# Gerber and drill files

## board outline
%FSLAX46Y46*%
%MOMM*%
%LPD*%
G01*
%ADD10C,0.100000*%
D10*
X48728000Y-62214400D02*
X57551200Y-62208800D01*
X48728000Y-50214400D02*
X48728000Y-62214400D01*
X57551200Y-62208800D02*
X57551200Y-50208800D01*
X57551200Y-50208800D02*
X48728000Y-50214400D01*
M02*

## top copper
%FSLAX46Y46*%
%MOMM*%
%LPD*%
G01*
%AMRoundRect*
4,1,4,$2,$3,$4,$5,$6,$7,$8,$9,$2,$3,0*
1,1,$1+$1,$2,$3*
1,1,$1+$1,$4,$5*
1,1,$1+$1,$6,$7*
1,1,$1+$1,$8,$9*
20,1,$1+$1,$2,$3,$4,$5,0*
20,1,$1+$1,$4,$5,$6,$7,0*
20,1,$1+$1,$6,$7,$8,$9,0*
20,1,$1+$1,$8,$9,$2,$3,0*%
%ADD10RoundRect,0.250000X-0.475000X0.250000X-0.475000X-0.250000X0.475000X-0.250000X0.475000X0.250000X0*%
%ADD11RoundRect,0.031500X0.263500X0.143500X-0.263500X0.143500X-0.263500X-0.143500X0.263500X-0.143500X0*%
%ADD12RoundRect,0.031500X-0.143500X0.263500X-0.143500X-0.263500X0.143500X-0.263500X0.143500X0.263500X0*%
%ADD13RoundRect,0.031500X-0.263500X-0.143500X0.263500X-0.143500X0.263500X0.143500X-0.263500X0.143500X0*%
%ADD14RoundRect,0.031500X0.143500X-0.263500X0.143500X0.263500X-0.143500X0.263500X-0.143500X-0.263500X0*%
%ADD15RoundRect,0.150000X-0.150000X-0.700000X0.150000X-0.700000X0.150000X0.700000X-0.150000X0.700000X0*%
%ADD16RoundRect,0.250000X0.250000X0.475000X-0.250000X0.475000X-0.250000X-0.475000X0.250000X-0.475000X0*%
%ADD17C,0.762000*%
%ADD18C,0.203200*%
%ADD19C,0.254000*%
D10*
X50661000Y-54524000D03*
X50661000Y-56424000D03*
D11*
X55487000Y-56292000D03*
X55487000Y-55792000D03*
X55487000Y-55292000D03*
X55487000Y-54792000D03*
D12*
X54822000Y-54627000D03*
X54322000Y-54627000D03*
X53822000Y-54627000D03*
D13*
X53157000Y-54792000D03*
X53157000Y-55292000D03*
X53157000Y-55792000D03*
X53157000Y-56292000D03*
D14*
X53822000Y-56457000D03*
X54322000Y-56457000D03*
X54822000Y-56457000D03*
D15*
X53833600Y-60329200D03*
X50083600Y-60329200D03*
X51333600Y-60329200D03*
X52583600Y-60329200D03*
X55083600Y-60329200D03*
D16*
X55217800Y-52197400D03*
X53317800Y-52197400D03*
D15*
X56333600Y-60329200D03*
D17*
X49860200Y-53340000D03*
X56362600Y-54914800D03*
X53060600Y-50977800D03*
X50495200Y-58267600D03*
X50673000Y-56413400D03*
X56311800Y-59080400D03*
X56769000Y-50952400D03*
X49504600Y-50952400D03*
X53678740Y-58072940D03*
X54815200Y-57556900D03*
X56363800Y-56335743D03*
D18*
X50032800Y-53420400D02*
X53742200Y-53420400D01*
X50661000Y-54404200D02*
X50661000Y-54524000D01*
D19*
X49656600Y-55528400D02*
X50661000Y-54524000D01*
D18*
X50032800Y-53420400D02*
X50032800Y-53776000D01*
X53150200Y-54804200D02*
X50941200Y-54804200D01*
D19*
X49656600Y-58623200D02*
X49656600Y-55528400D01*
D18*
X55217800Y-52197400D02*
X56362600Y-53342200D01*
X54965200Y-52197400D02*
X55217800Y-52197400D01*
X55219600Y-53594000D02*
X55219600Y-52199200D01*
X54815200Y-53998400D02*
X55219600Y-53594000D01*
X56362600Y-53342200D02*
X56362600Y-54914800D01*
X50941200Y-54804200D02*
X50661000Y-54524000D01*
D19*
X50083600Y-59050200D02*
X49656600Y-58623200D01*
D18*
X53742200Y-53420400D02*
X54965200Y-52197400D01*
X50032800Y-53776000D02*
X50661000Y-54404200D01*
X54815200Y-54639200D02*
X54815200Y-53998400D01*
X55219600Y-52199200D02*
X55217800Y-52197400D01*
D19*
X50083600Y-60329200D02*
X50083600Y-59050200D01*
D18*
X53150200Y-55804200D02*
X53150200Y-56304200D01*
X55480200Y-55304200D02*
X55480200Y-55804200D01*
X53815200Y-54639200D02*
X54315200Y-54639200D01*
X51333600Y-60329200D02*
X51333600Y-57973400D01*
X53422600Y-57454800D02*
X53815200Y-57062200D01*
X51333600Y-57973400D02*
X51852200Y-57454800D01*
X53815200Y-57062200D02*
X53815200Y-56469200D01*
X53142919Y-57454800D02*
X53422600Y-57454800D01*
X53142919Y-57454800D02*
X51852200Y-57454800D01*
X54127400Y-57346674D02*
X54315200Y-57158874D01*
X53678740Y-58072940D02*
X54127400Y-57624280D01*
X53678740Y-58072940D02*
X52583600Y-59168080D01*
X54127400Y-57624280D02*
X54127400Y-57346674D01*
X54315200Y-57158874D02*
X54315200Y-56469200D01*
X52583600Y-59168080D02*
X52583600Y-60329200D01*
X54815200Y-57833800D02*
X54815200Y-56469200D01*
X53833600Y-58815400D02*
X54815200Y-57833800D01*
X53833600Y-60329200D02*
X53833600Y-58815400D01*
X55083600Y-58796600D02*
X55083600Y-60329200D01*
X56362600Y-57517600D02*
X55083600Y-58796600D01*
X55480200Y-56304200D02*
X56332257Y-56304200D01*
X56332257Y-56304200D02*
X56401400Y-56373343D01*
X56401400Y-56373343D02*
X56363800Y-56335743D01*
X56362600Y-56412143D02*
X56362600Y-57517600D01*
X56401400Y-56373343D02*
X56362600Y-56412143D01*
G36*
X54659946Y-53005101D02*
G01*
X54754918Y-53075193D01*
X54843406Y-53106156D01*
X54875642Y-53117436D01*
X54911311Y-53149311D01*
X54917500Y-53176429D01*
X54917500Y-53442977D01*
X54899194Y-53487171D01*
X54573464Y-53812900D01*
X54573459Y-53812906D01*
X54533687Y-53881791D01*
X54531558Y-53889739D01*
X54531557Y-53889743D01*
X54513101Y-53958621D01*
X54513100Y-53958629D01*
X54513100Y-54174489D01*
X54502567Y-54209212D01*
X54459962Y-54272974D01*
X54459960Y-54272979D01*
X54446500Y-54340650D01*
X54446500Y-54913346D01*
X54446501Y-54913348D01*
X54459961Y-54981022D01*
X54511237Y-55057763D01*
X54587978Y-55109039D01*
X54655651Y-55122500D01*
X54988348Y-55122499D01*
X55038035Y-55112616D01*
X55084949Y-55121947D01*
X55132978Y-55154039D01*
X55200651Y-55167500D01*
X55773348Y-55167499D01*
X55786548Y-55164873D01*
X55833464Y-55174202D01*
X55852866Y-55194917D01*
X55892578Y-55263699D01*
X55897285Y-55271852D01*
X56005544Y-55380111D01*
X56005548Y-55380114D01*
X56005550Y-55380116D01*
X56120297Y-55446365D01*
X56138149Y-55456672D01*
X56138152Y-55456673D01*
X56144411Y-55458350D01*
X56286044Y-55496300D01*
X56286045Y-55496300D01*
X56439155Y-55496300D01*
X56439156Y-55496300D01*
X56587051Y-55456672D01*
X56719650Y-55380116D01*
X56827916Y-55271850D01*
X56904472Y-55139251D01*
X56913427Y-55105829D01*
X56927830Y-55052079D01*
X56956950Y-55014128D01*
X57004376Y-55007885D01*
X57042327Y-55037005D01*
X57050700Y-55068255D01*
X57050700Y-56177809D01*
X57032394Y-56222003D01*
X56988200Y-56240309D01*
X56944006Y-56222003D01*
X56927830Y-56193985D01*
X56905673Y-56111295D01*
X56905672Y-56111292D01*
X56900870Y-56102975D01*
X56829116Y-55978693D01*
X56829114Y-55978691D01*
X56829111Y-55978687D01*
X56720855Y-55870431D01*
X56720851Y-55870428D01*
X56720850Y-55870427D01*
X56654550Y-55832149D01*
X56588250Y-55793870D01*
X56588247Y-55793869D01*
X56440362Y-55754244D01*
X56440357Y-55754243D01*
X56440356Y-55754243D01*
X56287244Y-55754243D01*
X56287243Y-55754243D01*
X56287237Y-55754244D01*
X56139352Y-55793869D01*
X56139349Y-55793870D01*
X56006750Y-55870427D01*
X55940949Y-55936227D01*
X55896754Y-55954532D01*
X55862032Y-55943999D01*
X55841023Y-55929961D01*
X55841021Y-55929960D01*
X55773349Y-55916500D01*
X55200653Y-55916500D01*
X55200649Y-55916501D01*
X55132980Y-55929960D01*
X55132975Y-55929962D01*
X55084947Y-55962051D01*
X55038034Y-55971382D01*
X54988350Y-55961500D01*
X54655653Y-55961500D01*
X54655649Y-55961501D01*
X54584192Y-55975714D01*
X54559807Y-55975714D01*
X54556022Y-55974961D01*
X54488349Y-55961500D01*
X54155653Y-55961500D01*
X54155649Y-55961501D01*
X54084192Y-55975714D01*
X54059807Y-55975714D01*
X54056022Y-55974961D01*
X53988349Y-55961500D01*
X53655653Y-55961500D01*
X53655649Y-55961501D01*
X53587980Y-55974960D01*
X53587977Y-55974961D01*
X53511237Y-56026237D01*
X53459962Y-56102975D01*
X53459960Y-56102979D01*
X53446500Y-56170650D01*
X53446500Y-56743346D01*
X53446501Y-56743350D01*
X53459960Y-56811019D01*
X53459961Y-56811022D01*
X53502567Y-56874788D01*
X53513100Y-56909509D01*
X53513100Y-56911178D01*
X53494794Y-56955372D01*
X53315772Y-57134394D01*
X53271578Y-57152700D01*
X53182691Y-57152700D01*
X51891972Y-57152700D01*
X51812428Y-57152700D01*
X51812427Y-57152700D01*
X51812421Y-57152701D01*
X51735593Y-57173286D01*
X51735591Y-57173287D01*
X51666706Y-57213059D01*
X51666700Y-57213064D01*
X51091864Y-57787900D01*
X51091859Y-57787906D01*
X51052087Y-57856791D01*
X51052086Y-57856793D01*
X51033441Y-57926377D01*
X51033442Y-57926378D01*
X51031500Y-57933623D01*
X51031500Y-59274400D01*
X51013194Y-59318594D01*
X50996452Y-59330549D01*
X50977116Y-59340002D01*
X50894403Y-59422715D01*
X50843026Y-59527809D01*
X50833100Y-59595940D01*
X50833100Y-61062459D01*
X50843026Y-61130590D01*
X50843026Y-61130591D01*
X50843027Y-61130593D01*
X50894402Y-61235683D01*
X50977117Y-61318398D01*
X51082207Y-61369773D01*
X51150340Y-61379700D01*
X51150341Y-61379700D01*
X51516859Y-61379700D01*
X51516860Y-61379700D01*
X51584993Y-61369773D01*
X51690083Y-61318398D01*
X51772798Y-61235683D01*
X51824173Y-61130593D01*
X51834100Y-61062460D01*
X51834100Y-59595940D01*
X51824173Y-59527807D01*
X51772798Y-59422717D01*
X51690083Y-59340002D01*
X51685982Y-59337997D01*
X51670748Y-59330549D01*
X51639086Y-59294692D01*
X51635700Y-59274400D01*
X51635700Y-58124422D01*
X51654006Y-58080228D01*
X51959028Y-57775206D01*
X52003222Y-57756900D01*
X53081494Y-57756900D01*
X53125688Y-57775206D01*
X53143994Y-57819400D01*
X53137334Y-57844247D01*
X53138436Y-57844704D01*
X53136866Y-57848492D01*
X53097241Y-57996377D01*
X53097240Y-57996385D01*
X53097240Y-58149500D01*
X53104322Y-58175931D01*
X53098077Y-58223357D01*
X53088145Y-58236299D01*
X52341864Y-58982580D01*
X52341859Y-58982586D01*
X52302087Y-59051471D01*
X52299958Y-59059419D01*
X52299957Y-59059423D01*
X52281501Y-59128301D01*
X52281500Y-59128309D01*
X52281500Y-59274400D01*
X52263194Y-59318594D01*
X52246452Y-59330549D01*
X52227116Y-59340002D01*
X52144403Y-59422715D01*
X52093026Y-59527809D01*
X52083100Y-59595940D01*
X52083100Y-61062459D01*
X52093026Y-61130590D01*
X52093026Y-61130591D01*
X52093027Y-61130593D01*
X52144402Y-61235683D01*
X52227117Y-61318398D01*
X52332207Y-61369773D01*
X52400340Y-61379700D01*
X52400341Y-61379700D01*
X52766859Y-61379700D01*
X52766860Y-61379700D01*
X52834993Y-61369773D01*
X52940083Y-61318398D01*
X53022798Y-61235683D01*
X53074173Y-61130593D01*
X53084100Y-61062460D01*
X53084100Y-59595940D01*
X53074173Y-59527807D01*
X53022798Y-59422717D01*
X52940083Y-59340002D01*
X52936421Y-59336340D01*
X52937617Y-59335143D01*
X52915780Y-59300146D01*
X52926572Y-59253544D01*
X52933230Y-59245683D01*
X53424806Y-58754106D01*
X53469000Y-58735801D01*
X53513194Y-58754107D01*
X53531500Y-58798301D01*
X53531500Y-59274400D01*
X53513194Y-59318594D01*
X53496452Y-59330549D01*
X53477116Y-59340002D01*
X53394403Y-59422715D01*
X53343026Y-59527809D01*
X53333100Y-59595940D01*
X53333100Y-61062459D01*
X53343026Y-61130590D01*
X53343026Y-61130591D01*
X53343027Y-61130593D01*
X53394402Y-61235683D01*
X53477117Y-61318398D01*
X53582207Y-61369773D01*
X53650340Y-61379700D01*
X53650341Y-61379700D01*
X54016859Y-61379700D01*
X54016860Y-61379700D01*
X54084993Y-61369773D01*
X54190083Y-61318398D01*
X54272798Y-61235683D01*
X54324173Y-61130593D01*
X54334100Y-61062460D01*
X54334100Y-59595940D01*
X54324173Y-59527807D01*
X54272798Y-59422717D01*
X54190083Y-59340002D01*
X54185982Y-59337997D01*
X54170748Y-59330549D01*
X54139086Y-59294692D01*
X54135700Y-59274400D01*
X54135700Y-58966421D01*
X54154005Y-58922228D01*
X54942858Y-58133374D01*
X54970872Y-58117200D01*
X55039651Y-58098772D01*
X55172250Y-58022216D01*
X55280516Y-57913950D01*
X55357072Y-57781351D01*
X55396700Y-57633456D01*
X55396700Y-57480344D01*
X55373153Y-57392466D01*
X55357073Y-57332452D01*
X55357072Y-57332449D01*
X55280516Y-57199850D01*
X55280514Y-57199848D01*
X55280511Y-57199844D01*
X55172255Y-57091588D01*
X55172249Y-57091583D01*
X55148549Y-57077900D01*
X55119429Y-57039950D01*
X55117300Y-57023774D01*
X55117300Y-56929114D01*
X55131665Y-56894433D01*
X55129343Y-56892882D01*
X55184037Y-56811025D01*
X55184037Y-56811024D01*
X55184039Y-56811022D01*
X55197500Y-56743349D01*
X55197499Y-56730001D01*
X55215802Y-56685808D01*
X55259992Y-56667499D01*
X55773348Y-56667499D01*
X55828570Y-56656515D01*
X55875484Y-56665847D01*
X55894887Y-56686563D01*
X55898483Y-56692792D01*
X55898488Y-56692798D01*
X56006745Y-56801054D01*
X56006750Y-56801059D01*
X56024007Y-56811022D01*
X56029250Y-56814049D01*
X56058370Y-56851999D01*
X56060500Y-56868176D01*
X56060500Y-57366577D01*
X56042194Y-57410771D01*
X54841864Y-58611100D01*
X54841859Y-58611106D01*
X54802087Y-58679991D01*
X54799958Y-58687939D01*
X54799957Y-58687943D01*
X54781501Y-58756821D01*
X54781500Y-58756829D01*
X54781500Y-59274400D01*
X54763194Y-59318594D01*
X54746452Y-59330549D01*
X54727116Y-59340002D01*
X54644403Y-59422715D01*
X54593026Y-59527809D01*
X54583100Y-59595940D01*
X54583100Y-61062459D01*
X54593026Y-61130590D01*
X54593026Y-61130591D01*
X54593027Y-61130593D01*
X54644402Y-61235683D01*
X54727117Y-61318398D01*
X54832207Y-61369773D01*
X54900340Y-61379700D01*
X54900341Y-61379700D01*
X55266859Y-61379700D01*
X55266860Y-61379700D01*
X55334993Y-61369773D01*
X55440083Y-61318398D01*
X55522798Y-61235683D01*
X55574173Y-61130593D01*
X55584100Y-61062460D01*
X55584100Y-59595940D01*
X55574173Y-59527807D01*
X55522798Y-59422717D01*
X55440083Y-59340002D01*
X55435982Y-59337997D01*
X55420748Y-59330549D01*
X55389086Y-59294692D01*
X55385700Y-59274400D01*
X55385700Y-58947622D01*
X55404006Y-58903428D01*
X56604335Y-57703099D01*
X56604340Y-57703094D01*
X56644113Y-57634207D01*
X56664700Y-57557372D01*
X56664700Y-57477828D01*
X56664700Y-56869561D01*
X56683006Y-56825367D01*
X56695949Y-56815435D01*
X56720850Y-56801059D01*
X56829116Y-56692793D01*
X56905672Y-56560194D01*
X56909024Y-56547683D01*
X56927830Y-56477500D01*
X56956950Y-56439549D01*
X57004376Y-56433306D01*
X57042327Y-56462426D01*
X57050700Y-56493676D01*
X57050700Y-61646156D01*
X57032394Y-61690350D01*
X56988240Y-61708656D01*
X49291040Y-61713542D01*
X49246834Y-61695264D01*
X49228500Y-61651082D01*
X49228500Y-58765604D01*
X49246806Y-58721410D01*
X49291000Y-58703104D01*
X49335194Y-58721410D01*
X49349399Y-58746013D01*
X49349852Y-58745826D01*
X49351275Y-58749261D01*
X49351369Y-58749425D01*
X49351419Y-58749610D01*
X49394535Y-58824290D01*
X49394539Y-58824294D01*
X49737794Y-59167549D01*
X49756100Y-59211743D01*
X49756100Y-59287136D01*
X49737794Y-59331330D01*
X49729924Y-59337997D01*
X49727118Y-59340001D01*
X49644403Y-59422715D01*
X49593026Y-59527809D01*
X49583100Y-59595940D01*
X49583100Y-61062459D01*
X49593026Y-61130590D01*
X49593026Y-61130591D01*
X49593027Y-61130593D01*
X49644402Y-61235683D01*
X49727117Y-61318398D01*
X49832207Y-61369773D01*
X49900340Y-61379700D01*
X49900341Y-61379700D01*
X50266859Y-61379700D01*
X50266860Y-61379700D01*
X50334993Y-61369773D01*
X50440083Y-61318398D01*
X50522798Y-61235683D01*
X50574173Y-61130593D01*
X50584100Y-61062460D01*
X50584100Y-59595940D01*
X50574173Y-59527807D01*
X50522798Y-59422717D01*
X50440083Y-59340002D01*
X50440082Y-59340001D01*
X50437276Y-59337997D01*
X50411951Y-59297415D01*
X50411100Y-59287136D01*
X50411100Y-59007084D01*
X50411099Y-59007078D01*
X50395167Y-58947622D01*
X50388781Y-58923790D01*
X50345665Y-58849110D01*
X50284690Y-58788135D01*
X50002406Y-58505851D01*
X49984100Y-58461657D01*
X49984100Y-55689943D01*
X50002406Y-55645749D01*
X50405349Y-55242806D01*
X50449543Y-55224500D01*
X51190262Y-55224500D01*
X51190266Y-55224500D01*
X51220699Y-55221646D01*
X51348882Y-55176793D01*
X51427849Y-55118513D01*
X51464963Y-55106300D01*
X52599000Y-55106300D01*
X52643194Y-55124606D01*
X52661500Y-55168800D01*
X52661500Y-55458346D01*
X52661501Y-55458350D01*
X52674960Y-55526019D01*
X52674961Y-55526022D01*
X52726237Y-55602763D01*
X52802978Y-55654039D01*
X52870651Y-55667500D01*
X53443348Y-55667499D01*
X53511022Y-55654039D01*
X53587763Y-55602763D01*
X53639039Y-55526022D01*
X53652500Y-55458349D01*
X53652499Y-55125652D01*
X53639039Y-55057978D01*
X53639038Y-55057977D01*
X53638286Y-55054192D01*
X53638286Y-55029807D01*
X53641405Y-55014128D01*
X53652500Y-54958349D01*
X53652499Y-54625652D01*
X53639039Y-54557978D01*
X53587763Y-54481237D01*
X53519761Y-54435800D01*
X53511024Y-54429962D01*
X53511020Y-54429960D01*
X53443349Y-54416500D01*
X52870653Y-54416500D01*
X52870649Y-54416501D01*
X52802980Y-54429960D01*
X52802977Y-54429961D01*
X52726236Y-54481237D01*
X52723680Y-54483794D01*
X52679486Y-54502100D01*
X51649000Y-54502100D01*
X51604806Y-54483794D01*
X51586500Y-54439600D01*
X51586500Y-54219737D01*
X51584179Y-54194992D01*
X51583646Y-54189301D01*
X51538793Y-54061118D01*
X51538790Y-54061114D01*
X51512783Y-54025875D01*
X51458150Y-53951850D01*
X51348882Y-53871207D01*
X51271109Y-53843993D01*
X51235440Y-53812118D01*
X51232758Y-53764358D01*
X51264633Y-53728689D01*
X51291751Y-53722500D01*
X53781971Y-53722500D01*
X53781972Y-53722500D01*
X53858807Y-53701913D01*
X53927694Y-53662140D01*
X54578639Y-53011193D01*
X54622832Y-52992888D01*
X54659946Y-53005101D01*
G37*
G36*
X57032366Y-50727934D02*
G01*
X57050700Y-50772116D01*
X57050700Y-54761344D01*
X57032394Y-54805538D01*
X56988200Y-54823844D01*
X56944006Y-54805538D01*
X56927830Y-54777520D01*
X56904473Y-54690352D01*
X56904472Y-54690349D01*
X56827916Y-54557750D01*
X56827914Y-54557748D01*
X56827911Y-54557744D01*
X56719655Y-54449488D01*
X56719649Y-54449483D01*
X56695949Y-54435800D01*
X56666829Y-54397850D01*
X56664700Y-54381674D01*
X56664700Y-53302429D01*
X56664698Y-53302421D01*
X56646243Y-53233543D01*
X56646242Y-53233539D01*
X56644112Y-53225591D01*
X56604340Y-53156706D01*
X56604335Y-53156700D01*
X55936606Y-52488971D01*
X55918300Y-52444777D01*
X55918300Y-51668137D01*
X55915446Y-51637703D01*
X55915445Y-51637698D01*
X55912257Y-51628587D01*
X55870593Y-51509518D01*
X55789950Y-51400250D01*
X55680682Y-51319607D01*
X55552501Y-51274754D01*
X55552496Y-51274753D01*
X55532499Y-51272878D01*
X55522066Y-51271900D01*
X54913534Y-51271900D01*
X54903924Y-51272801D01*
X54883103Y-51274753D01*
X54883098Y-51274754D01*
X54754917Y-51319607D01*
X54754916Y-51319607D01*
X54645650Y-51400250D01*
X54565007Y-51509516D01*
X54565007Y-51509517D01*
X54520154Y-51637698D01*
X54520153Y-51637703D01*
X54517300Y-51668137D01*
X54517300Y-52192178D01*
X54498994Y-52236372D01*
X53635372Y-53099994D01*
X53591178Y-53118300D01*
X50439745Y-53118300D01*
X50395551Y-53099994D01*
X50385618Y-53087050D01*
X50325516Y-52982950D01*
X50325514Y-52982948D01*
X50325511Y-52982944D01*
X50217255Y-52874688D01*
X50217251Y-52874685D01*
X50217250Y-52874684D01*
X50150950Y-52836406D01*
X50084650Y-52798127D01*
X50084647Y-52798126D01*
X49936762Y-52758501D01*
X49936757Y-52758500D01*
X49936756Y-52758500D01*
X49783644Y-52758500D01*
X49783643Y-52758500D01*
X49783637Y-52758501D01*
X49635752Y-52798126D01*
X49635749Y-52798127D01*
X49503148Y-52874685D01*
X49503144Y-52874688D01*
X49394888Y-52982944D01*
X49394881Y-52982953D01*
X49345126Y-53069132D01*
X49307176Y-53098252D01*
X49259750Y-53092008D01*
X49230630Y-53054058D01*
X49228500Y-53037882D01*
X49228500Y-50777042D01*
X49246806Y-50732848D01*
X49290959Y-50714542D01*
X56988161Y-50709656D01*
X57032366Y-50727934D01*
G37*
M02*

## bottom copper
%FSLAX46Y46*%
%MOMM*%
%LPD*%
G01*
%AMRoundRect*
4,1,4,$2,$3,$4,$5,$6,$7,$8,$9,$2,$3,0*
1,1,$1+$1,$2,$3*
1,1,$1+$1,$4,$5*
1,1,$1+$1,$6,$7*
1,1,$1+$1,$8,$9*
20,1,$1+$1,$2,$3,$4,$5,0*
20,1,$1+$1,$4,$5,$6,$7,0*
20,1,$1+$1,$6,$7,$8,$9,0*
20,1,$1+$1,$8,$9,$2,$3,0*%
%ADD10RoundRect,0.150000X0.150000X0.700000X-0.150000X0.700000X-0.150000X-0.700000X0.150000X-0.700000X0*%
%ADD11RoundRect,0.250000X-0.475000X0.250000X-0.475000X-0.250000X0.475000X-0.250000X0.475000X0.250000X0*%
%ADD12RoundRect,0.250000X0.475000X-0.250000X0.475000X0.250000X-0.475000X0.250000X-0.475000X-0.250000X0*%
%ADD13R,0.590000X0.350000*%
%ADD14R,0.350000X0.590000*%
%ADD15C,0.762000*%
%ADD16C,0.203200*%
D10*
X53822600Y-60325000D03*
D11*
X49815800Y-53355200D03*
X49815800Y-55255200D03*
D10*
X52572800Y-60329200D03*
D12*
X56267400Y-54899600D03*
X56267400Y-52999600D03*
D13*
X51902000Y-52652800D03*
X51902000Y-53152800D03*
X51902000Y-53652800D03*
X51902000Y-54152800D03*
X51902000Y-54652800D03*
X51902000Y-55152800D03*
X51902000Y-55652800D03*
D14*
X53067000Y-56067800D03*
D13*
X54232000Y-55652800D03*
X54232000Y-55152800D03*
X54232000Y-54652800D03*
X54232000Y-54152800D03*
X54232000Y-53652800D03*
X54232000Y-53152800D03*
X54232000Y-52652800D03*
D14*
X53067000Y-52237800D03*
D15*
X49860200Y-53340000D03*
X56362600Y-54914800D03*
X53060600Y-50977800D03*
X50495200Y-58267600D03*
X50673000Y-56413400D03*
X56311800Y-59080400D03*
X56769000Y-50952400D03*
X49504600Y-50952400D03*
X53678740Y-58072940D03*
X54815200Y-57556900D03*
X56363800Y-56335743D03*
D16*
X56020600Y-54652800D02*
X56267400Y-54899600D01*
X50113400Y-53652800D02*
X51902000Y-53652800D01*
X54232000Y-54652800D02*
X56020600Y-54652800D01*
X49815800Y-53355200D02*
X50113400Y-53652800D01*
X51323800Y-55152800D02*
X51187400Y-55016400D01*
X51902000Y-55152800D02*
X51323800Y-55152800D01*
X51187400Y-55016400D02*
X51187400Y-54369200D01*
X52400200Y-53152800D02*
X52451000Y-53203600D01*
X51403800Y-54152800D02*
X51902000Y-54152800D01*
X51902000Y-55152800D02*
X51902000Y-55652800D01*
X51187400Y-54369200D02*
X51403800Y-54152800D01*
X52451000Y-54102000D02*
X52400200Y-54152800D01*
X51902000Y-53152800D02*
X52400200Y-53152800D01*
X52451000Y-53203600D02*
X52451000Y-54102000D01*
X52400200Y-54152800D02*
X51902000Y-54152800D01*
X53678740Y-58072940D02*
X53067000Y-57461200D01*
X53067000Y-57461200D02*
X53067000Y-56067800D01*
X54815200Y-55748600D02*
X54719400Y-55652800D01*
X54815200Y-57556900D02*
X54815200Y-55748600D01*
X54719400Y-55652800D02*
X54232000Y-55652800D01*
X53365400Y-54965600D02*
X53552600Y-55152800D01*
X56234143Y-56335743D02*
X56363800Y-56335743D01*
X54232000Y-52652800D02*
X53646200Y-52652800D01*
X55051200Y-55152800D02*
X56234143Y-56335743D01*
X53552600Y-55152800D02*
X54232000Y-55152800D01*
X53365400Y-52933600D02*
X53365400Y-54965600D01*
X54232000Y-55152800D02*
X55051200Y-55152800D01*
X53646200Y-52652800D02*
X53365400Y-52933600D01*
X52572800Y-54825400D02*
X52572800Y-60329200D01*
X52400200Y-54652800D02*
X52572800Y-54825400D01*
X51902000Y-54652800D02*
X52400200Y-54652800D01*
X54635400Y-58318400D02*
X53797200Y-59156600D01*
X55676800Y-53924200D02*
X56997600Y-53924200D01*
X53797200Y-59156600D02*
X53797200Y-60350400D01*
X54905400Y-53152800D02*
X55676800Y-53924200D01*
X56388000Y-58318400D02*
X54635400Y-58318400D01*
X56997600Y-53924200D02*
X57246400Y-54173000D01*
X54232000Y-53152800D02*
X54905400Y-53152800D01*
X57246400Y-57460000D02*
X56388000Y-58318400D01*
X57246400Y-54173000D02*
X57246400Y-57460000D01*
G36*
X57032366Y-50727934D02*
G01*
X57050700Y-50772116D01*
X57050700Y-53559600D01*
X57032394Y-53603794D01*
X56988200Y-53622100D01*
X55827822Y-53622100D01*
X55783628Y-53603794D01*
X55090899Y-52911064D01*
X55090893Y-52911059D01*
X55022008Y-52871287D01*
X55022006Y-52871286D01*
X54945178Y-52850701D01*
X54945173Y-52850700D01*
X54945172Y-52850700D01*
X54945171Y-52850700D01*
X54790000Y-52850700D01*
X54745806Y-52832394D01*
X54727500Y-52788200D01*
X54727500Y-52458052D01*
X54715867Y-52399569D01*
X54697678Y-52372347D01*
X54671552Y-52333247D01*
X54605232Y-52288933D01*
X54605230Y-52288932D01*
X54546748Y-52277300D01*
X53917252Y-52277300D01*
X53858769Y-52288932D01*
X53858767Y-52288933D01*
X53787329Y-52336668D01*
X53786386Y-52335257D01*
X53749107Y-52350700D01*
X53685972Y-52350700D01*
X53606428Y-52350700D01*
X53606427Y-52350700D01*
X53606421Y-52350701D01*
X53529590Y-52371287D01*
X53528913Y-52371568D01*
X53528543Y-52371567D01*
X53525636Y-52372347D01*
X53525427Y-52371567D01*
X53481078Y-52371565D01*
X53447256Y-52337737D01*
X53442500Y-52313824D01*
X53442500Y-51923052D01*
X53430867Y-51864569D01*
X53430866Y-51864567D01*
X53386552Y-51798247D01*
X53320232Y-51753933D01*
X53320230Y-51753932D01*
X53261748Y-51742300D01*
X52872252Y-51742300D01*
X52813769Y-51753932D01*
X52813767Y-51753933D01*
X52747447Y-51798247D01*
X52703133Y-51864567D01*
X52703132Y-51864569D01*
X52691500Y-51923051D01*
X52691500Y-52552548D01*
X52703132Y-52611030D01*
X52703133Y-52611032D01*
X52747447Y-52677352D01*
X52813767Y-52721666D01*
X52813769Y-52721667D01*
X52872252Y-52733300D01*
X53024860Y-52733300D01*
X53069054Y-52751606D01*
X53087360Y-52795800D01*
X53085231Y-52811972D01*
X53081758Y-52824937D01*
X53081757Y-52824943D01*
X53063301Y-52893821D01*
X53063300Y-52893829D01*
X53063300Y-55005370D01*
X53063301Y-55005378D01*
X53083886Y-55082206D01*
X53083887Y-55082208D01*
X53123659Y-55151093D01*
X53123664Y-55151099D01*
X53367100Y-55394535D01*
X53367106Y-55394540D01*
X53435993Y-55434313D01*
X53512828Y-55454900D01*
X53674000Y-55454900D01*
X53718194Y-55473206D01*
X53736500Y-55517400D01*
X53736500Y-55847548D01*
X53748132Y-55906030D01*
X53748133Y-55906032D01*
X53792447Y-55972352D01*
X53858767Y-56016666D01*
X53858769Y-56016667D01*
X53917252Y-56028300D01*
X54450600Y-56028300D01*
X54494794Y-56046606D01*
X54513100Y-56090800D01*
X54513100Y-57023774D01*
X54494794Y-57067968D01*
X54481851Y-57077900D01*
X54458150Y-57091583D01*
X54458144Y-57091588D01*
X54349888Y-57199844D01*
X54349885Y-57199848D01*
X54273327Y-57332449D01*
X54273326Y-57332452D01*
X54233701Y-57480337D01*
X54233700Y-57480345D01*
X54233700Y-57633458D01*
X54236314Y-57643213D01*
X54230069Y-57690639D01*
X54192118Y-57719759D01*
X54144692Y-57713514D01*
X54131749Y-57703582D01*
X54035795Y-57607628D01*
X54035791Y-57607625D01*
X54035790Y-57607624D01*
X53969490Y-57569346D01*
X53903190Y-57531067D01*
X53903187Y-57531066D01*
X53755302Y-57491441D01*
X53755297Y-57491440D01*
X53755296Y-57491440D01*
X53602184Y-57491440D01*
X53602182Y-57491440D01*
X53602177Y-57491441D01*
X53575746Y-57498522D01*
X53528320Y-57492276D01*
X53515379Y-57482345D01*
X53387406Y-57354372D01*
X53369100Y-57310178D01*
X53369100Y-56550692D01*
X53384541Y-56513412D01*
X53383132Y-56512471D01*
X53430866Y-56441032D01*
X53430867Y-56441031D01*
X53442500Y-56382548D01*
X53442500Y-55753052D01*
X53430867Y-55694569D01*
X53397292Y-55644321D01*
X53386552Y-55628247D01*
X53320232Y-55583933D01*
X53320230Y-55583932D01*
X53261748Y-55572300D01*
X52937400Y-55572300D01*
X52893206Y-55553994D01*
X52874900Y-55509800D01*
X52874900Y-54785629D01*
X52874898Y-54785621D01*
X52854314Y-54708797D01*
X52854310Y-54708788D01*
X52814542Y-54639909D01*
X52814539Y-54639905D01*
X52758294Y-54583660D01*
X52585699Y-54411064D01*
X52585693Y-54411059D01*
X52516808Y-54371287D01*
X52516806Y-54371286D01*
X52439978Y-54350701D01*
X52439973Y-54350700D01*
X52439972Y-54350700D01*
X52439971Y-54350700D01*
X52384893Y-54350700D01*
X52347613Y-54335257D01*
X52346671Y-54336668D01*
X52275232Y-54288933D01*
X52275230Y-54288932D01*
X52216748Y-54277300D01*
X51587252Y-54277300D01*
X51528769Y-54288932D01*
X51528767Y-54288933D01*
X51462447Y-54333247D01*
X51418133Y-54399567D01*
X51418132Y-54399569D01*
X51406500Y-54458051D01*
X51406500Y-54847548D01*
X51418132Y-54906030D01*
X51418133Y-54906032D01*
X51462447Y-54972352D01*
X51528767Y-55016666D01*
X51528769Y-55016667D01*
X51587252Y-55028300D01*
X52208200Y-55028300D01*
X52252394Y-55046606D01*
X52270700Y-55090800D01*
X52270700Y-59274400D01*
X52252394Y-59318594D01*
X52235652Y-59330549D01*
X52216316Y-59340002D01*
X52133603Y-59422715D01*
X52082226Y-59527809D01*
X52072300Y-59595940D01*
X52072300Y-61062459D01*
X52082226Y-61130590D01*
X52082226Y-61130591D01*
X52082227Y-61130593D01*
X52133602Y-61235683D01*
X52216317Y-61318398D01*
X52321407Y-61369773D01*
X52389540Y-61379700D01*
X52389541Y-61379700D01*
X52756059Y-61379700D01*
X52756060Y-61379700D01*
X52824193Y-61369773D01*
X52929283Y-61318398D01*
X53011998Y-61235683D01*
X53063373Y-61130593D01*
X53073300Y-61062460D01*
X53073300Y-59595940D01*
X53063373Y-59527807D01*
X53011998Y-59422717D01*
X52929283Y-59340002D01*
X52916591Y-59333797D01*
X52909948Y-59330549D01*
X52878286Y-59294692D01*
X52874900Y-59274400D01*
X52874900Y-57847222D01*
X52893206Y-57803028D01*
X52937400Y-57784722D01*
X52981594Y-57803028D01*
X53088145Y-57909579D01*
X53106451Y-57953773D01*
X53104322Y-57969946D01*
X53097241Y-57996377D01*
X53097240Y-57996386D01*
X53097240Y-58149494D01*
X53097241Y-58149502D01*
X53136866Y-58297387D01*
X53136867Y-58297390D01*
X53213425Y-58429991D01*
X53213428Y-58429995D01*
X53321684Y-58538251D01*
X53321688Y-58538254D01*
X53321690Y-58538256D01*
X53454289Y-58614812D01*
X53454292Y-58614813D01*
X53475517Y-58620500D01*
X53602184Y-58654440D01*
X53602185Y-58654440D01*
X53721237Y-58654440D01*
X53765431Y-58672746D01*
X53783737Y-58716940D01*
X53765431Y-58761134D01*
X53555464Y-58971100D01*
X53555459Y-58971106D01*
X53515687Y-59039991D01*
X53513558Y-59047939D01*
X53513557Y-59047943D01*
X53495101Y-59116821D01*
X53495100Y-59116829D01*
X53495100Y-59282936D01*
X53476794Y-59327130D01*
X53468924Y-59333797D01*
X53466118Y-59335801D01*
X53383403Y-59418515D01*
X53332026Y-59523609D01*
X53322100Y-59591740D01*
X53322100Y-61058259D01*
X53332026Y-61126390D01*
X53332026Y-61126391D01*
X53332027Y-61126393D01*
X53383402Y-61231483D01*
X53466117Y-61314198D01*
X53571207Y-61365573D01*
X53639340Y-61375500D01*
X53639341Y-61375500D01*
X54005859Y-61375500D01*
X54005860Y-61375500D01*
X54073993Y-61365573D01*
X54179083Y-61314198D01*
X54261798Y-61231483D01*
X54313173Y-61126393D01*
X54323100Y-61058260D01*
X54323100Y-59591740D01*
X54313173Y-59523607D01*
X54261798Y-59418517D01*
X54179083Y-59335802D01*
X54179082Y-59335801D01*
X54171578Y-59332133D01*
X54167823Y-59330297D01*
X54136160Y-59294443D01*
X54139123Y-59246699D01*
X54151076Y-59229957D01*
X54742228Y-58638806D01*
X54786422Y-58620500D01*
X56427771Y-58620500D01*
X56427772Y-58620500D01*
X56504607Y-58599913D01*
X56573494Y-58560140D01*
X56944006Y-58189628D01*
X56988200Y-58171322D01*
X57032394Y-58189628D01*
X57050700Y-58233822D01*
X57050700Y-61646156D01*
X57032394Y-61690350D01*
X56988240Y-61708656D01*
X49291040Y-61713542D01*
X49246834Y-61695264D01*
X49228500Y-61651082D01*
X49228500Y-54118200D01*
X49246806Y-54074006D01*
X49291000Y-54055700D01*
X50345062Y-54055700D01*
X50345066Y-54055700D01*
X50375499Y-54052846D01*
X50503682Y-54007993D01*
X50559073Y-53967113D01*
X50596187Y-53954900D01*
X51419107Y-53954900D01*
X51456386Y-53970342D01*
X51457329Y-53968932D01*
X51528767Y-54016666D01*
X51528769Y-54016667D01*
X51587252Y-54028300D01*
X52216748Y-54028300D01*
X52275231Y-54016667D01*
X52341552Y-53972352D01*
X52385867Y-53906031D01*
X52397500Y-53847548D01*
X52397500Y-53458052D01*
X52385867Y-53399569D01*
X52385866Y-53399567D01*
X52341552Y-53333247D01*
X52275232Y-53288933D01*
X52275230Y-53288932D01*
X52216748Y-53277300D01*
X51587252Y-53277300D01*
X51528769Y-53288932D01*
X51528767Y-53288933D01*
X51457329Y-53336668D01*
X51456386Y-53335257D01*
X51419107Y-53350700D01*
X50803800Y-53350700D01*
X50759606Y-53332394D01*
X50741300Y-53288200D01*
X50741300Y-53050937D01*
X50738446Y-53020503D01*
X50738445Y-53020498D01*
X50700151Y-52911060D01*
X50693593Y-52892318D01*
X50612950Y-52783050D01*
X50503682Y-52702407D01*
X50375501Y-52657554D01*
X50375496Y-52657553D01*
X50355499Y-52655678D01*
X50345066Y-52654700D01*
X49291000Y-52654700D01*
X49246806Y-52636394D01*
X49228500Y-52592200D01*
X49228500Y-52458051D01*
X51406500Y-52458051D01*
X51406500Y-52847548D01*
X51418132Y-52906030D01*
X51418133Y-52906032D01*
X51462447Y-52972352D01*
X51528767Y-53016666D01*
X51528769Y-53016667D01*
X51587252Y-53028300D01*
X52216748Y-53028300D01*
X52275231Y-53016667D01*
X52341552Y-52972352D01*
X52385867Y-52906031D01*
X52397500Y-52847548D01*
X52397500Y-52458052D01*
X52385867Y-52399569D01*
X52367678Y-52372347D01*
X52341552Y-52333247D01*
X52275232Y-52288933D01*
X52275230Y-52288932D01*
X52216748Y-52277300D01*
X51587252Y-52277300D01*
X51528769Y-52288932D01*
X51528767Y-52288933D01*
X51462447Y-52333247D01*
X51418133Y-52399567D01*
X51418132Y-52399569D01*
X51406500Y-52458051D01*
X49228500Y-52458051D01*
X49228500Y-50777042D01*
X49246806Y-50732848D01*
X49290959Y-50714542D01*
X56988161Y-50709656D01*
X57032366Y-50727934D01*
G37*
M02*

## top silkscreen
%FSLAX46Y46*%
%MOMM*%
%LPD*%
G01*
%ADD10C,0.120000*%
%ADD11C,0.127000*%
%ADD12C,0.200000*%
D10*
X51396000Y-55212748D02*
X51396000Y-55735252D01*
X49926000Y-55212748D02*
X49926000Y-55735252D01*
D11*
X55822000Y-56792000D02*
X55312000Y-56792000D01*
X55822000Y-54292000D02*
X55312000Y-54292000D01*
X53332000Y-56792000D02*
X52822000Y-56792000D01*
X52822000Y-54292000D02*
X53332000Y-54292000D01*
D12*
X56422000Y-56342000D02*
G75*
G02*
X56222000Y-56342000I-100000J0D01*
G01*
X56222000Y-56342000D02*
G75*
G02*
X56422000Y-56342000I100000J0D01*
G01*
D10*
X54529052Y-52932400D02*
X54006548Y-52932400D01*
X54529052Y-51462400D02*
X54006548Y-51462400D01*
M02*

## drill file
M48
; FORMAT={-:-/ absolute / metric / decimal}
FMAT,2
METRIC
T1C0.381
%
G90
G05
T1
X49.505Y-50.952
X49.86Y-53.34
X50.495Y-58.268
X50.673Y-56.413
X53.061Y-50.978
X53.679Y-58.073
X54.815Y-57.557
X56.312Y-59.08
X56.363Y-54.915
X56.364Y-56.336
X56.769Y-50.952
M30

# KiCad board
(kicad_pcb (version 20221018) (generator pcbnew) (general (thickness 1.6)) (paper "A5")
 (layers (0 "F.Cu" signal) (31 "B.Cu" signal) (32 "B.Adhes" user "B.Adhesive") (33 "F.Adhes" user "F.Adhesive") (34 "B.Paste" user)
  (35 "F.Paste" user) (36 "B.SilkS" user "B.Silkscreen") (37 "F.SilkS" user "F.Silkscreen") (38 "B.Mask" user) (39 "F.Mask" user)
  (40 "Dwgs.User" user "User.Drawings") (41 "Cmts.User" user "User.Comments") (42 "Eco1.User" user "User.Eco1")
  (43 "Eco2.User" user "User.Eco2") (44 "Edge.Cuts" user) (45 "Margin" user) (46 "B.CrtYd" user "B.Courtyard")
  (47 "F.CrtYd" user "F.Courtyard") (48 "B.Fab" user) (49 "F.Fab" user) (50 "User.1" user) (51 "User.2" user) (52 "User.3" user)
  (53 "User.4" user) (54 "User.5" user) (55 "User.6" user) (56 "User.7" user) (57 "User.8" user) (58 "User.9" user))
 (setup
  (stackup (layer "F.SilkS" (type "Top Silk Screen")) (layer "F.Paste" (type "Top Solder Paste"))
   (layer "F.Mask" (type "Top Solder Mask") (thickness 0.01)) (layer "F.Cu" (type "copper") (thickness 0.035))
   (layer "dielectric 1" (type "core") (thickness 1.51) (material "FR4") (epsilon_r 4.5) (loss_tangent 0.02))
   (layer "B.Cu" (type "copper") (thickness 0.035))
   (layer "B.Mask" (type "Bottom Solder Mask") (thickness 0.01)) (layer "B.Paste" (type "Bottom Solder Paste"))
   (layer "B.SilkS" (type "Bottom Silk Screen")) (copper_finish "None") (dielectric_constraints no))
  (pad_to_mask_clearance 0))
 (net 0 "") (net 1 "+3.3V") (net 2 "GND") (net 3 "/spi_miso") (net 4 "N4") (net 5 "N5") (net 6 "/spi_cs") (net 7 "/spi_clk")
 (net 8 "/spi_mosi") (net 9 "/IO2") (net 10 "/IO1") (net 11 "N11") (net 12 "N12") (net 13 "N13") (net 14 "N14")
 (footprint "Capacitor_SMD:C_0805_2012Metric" (layer "F.Cu") (at 50.661 55.474 -90)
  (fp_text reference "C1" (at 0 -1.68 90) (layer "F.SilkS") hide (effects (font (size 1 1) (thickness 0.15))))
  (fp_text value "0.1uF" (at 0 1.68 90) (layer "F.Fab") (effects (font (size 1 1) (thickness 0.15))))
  (fp_line (start -0.261252 -0.735) (end 0.261252 -0.735) (stroke (width 0.12) (type solid)) (layer "F.SilkS"))
  (fp_line (start -0.261252 0.735) (end 0.261252 0.735) (stroke (width 0.12) (type solid)) (layer "F.SilkS"))
  (pad "1" smd roundrect (at -0.95 0 270) (size 1 1.45) (layers "F.Cu" "F.Paste" "F.Mask") (roundrect_rratio 0.25) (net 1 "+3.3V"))
  (pad "2" smd roundrect (at 0.95 0 270) (size 1 1.45) (layers "F.Cu" "F.Paste" "F.Mask") (roundrect_rratio 0.25) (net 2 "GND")))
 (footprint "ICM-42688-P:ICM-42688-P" (layer "F.Cu") (at 54.322 55.542 180)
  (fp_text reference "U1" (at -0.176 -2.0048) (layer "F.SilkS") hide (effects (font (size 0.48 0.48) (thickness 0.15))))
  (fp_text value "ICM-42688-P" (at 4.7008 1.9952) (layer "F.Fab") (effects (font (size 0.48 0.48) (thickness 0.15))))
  (fp_line (start -1.5 -1.25) (end -0.99 -1.25) (stroke (width 0.127) (type solid)) (layer "F.SilkS"))
  (fp_line (start -1.5 1.25) (end -0.99 1.25) (stroke (width 0.127) (type solid)) (layer "F.SilkS"))
  (fp_line (start 0.99 -1.25) (end 1.5 -1.25) (stroke (width 0.127) (type solid)) (layer "F.SilkS"))
  (fp_line (start 1.5 1.25) (end 0.99 1.25) (stroke (width 0.127) (type solid)) (layer "F.SilkS"))
  (fp_circle (center -2 -0.8) (end -1.9 -0.8) (stroke (width 0.2) (type solid)) (fill none) (layer "F.SilkS"))
  (pad "1" smd roundrect (at -1.165 -0.75 180) (size 0.59 0.35) (layers "F.Cu" "F.Paste") (roundrect_rratio 0.09) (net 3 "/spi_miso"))
  (pad "2" smd roundrect (at -1.165 -0.25 180) (size 0.59 0.35) (layers "F.Cu" "F.Paste") (roundrect_rratio 0.09) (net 2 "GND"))
  (pad "3" smd roundrect (at -1.165 0.25 180) (size 0.59 0.35) (layers "F.Cu" "F.Paste") (roundrect_rratio 0.09) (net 2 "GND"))
  (pad "4" smd roundrect (at -1.165 0.75 180) (size 0.59 0.35) (layers "F.Cu" "F.Paste") (roundrect_rratio 0.09) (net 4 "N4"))
  (pad "5" smd roundrect (at -0.5 0.915 270) (size 0.59 0.35) (layers "F.Cu" "F.Paste") (roundrect_rratio 0.09) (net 1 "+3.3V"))
  (pad "6" smd roundrect (at 0 0.915 270) (size 0.59 0.35) (layers "F.Cu" "F.Paste") (roundrect_rratio 0.09) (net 2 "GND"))
  (pad "7" smd roundrect (at 0.5 0.915 270) (size 0.59 0.35) (layers "F.Cu" "F.Paste") (roundrect_rratio 0.09) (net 2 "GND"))
  (pad "8" smd roundrect (at 1.165 0.75) (size 0.59 0.35) (layers "F.Cu" "F.Paste") (roundrect_rratio 0.09) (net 1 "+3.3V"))
  (pad "9" smd roundrect (at 1.165 0.25) (size 0.59 0.35) (layers "F.Cu" "F.Paste") (roundrect_rratio 0.09) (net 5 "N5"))
  (pad "10" smd roundrect (at 1.165 -0.25) (size 0.59 0.35) (layers "F.Cu" "F.Paste") (roundrect_rratio 0.09) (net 2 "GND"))
  (pad "11" smd roundrect (at 1.165 -0.75) (size 0.59 0.35) (layers "F.Cu" "F.Paste") (roundrect_rratio 0.09) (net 2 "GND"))
  (pad "12" smd roundrect (at 0.5 -0.915 90) (size 0.59 0.35) (layers "F.Cu" "F.Paste") (roundrect_rratio 0.09) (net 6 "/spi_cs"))
  (pad "13" smd roundrect (at 0 -0.915 90) (size 0.59 0.35) (layers "F.Cu" "F.Paste") (roundrect_rratio 0.09) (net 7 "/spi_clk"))
  (pad "14" smd roundrect (at -0.5 -0.915 90) (size 0.59 0.35) (layers "F.Cu" "F.Paste") (roundrect_rratio 0.09) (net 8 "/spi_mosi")))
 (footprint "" (layer "F.Cu") (at 53.8336 60.3292)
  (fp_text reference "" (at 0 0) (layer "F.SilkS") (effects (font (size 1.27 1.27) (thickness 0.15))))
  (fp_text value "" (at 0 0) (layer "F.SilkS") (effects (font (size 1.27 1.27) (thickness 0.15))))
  (pad "4" smd roundrect (at 0 0) (size 0.6 1.7) (layers "F.Cu" "F.Paste" "F.Mask") (roundrect_rratio 0.25) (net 8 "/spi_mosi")))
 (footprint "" (layer "F.Cu") (at 50.0836 60.3292)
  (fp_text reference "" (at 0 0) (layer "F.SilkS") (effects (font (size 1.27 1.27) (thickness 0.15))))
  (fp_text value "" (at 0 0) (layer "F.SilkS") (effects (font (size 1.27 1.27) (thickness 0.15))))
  (pad "1" smd roundrect (at 0 0) (size 0.6 1.7) (layers "F.Cu" "F.Paste" "F.Mask") (roundrect_rratio 0.25) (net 1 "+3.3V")))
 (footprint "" (layer "F.Cu") (at 51.3336 60.3292)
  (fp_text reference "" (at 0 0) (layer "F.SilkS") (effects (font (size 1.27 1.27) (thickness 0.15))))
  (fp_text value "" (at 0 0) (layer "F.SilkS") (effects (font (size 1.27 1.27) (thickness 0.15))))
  (pad "2" smd roundrect (at 0 0) (size 0.6 1.7) (layers "F.Cu" "F.Paste" "F.Mask") (roundrect_rratio 0.25) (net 6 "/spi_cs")))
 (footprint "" (layer "F.Cu") (at 52.5836 60.3292)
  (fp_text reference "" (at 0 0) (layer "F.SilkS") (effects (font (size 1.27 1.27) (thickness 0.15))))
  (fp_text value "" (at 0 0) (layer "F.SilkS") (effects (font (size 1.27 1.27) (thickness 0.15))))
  (pad "3" smd roundrect (at 0 0) (size 0.6 1.7) (layers "F.Cu" "F.Paste" "F.Mask") (roundrect_rratio 0.25) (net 7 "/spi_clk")))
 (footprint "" (layer "F.Cu") (at 55.0836 60.3292)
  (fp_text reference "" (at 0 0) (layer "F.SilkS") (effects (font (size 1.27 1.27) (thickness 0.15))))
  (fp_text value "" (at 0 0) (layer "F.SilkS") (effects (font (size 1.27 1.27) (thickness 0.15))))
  (pad "5" smd roundrect (at 0 0) (size 0.6 1.7) (layers "F.Cu" "F.Paste" "F.Mask") (roundrect_rratio 0.25) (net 3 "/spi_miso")))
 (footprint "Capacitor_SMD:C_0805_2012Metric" (layer "F.Cu") (at 54.2678 52.1974 180)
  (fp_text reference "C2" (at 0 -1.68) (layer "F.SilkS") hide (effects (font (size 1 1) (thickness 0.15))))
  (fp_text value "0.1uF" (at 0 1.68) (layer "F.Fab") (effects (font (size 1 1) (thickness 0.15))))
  (fp_line (start -0.261252 -0.735) (end 0.261252 -0.735) (stroke (width 0.12) (type solid)) (layer "F.SilkS"))
  (fp_line (start -0.261252 0.735) (end 0.261252 0.735) (stroke (width 0.12) (type solid)) (layer "F.SilkS"))
  (pad "1" smd roundrect (at -0.95 0 180) (size 1 1.45) (layers "F.Cu" "F.Paste" "F.Mask") (roundrect_rratio 0.25) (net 1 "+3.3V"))
  (pad "2" smd roundrect (at 0.95 0 180) (size 1 1.45) (layers "F.Cu" "F.Paste" "F.Mask") (roundrect_rratio 0.25) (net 2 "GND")))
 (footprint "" (layer "F.Cu") (at 56.3336 60.3292)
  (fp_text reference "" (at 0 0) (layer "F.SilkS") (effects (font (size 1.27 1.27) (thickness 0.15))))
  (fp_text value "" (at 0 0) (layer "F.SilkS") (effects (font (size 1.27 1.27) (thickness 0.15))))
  (pad "6" smd roundrect (at 0 0) (size 0.6 1.7) (layers "F.Cu" "F.Paste" "F.Mask") (roundrect_rratio 0.25) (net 2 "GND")))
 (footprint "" (layer "B.Cu") (at 53.8226 60.325 180)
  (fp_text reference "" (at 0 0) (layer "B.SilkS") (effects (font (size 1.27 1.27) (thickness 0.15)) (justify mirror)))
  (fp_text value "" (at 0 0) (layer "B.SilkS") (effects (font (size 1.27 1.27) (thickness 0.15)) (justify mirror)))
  (pad "3" smd roundrect (at 0 0 180) (size 0.6 1.7) (layers "B.Cu" "B.Paste" "B.Mask") (roundrect_rratio 0.25) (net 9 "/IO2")))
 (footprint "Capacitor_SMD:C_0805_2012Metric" (layer "B.Cu") (at 49.8158 54.3052 -90)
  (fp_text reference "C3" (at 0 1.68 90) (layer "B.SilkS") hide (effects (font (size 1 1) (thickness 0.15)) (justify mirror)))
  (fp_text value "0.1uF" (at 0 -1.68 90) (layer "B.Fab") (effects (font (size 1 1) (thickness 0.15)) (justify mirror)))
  (pad "1" smd roundrect (at -0.95 0 270) (size 1 1.45) (layers "B.Cu" "B.Paste" "B.Mask") (roundrect_rratio 0.25) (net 1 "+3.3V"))
  (pad "2" smd roundrect (at 0.95 0 270) (size 1 1.45) (layers "B.Cu" "B.Paste" "B.Mask") (roundrect_rratio 0.25) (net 2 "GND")))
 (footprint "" (layer "B.Cu") (at 52.5728 60.3292 180)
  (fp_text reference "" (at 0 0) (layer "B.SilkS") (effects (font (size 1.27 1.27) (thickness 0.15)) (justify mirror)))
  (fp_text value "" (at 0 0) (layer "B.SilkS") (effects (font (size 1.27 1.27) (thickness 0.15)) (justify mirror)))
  (pad "2" smd roundrect (at 0 0 180) (size 0.6 1.7) (layers "B.Cu" "B.Paste" "B.Mask") (roundrect_rratio 0.25) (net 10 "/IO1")))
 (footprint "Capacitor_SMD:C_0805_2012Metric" (layer "B.Cu") (at 56.2674 53.9496 90)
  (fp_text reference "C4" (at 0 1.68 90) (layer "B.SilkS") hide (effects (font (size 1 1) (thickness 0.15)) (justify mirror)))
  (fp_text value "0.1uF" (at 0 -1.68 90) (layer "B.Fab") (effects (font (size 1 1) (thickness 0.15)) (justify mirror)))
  (pad "1" smd roundrect (at -0.95 0 90) (size 1 1.45) (layers "B.Cu" "B.Paste" "B.Mask") (roundrect_rratio 0.25) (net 1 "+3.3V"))
  (pad "2" smd roundrect (at 0.95 0 90) (size 1 1.45) (layers "B.Cu" "B.Paste" "B.Mask") (roundrect_rratio 0.25) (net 2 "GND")))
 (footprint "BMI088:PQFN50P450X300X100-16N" (layer "B.Cu") (at 53.067 54.1528 -90)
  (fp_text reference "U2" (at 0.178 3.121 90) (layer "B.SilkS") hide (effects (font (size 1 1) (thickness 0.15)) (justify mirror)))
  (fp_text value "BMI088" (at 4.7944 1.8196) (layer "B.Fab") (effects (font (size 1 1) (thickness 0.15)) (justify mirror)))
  (pad "1" smd rect (at -1.5 1.165) (size 0.59 0.35) (layers "B.Cu" "B.Paste" "B.Mask") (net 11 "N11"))
  (pad "2" smd rect (at -1 1.165) (size 0.59 0.35) (layers "B.Cu" "B.Paste" "B.Mask") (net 2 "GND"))
  (pad "3" smd rect (at -0.5 1.165) (size 0.59 0.35) (layers "B.Cu" "B.Paste" "B.Mask") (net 1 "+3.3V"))
  (pad "4" smd rect (at 0 1.165) (size 0.59 0.35) (layers "B.Cu" "B.Paste" "B.Mask") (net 2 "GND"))
  (pad "5" smd rect (at 0.5 1.165) (size 0.59 0.35) (layers "B.Cu" "B.Paste" "B.Mask") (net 10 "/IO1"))
  (pad "6" smd rect (at 1 1.165) (size 0.59 0.35) (layers "B.Cu" "B.Paste" "B.Mask") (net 2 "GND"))
  (pad "7" smd rect (at 1.5 1.165) (size 0.59 0.35) (layers "B.Cu" "B.Paste" "B.Mask") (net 2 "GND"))
  (pad "8" smd rect (at 1.915 0 90) (size 0.59 0.35) (layers "B.Cu" "B.Paste" "B.Mask") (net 7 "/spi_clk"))
  (pad "9" smd rect (at 1.5 -1.165 180) (size 0.59 0.35) (layers "B.Cu" "B.Paste" "B.Mask") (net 8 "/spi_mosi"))
  (pad "10" smd rect (at 1 -1.165 180) (size 0.59 0.35) (layers "B.Cu" "B.Paste" "B.Mask") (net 3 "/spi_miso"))
  (pad "11" smd rect (at 0.5 -1.165 180) (size 0.59 0.35) (layers "B.Cu" "B.Paste" "B.Mask") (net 1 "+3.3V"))
  (pad "12" smd rect (at 0 -1.165 180) (size 0.59 0.35) (layers "B.Cu" "B.Paste" "B.Mask") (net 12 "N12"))
  (pad "13" smd rect (at -0.5 -1.165 180) (size 0.59 0.35) (layers "B.Cu" "B.Paste" "B.Mask") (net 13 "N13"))
  (pad "14" smd rect (at -1 -1.165 180) (size 0.59 0.35) (layers "B.Cu" "B.Paste" "B.Mask") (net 9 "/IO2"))
  (pad "15" smd rect (at -1.5 -1.165 180) (size 0.59 0.35) (layers "B.Cu" "B.Paste" "B.Mask") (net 3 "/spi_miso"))
  (pad "16" smd rect (at -1.915 0 270) (size 0.59 0.35) (layers "B.Cu" "B.Paste" "B.Mask") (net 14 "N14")))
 (gr_line locked (start 48.728 62.2144) (end 57.5512 62.2088) (stroke (width 0.1) (type default)) (layer "Edge.Cuts"))
 (gr_line locked (start 48.728 50.2144) (end 48.728 62.2144) (stroke (width 0.1) (type default)) (layer "Edge.Cuts"))
 (gr_line locked (start 57.5512 62.2088) (end 57.5512 50.2088) (stroke (width 0.1) (type default)) (layer "Edge.Cuts"))
 (gr_line locked (start 57.5512 50.2088) (end 48.728 50.2144) (stroke (width 0.1) (type default)) (layer "Edge.Cuts"))
 (segment (start 50.0328 53.4204) (end 53.7422 53.4204) (width 0.2032) (layer "F.Cu") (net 1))
 (segment (start 50.661 54.4042) (end 50.661 54.524) (width 0.2032) (layer "F.Cu") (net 1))
 (segment (start 49.6566 55.5284) (end 50.661 54.524) (width 0.254) (layer "F.Cu") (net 1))
 (segment (start 50.0328 53.4204) (end 50.0328 53.776) (width 0.2032) (layer "F.Cu") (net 1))
 (segment (start 53.1502 54.8042) (end 50.9412 54.8042) (width 0.2032) (layer "F.Cu") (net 1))
 (segment (start 49.6566 58.6232) (end 49.6566 55.5284) (width 0.254) (layer "F.Cu") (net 1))
 (segment (start 55.2178 52.1974) (end 56.3626 53.3422) (width 0.2032) (layer "F.Cu") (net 1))
 (segment (start 54.9652 52.1974) (end 55.2178 52.1974) (width 0.2032) (layer "F.Cu") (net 1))
 (segment (start 55.2196 53.594) (end 55.2196 52.1992) (width 0.2032) (layer "F.Cu") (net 1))
 (segment (start 54.8152 53.9984) (end 55.2196 53.594) (width 0.2032) (layer "F.Cu") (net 1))
 (segment (start 56.3626 53.3422) (end 56.3626 54.9148) (width 0.2032) (layer "F.Cu") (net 1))
 (segment (start 50.9412 54.8042) (end 50.661 54.524) (width 0.2032) (layer "F.Cu") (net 1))
 (segment (start 50.0836 59.0502) (end 49.6566 58.6232) (width 0.254) (layer "F.Cu") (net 1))
 (segment (start 53.7422 53.4204) (end 54.9652 52.1974) (width 0.2032) (layer "F.Cu") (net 1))
 (segment (start 50.0328 53.776) (end 50.661 54.4042) (width 0.2032) (layer "F.Cu") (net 1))
 (segment (start 54.8152 54.6392) (end 54.8152 53.9984) (width 0.2032) (layer "F.Cu") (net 1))
 (segment (start 55.2196 52.1992) (end 55.2178 52.1974) (width 0.2032) (layer "F.Cu") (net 1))
 (segment (start 50.0836 60.3292) (end 50.0836 59.0502) (width 0.254) (layer "F.Cu") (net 1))
 (via (at 49.8602 53.34) (size 0.762) (drill 0.381) (layers "F.Cu" "B.Cu") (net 1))
 (via (at 56.3626 54.9148) (size 0.762) (drill 0.381) (layers "F.Cu" "B.Cu") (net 1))
 (segment (start 56.0206 54.6528) (end 56.2674 54.8996) (width 0.2032) (layer "B.Cu") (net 1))
 (segment (start 50.1134 53.6528) (end 51.902 53.6528) (width 0.2032) (layer "B.Cu") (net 1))
 (segment (start 54.232 54.6528) (end 56.0206 54.6528) (width 0.2032) (layer "B.Cu") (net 1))
 (segment (start 49.8158 53.3552) (end 50.1134 53.6528) (width 0.2032) (layer "B.Cu") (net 1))
 (segment (start 53.1502 55.8042) (end 53.1502 56.3042) (width 0.2032) (layer "F.Cu") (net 2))
 (segment (start 55.4802 55.3042) (end 55.4802 55.8042) (width 0.2032) (layer "F.Cu") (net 2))
 (segment (start 53.8152 54.6392) (end 54.3152 54.6392) (width 0.2032) (layer "F.Cu") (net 2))
 (via (at 53.0606 50.9778) (size 0.762) (drill 0.381) (layers "F.Cu" "B.Cu") (free) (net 2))
 (via (at 50.4952 58.2676) (size 0.762) (drill 0.381) (layers "F.Cu" "B.Cu") (free) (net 2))
 (via (at 50.673 56.4134) (size 0.762) (drill 0.381) (layers "F.Cu" "B.Cu") (free) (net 2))
 (via (at 56.3118 59.0804) (size 0.762) (drill 0.381) (layers "F.Cu" "B.Cu") (free) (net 2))
 (via (at 56.769 50.9524) (size 0.762) (drill 0.381) (layers "F.Cu" "B.Cu") (free) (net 2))
 (via (at 49.5046 50.9524) (size 0.762) (drill 0.381) (layers "F.Cu" "B.Cu") (free) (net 2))
 (segment (start 51.3238 55.1528) (end 51.1874 55.0164) (width 0.2032) (layer "B.Cu") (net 2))
 (segment (start 51.902 55.1528) (end 51.3238 55.1528) (width 0.2032) (layer "B.Cu") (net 2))
 (segment (start 51.1874 55.0164) (end 51.1874 54.3692) (width 0.2032) (layer "B.Cu") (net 2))
 (segment (start 52.4002 53.1528) (end 52.451 53.2036) (width 0.2032) (layer "B.Cu") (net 2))
 (segment (start 51.4038 54.1528) (end 51.902 54.1528) (width 0.2032) (layer "B.Cu") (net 2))
 (segment (start 51.902 55.1528) (end 51.902 55.6528) (width 0.2032) (layer "B.Cu") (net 2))
 (segment (start 51.1874 54.3692) (end 51.4038 54.1528) (width 0.2032) (layer "B.Cu") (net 2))
 (segment (start 52.451 54.102) (end 52.4002 54.1528) (width 0.2032) (layer "B.Cu") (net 2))
 (segment (start 51.902 53.1528) (end 52.4002 53.1528) (width 0.2032) (layer "B.Cu") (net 2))
 (segment (start 52.451 53.2036) (end 52.451 54.102) (width 0.2032) (layer "B.Cu") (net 2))
 (segment (start 52.4002 54.1528) (end 51.902 54.1528) (width 0.2032) (layer "B.Cu") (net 2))
 (segment (start 51.3336 60.3292) (end 51.3336 57.9734) (width 0.2032) (layer "F.Cu") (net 6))
 (segment (start 53.4226 57.4548) (end 53.8152 57.0622) (width 0.2032) (layer "F.Cu") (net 6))
 (segment (start 51.3336 57.9734) (end 51.8522 57.4548) (width 0.2032) (layer "F.Cu") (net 6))
 (segment (start 53.8152 57.0622) (end 53.8152 56.4692) (width 0.2032) (layer "F.Cu") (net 6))
 (segment (start 53.142919 57.4548) (end 53.4226 57.4548) (width 0.2032) (layer "F.Cu") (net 6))
 (segment (start 53.142919 57.4548) (end 51.8522 57.4548) (width 0.2032) (layer "F.Cu") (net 6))
 (segment (start 54.1274 57.346674) (end 54.3152 57.158874) (width 0.2032) (layer "F.Cu") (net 7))
 (segment (start 53.67874 58.07294) (end 54.1274 57.62428) (width 0.2032) (layer "F.Cu") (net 7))
 (segment (start 53.67874 58.07294) (end 52.5836 59.16808) (width 0.2032) (layer "F.Cu") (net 7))
 (segment (start 54.1274 57.62428) (end 54.1274 57.346674) (width 0.2032) (layer "F.Cu") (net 7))
 (segment (start 54.3152 57.158874) (end 54.3152 56.4692) (width 0.2032) (layer "F.Cu") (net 7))
 (segment (start 52.5836 59.16808) (end 52.5836 60.3292) (width 0.2032) (layer "F.Cu") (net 7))
 (via (at 53.67874 58.07294) (size 0.762) (drill 0.381) (layers "F.Cu" "B.Cu") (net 7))
 (segment (start 53.67874 58.07294) (end 53.067 57.4612) (width 0.2032) (layer "B.Cu") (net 7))
 (segment (start 53.067 57.4612) (end 53.067 56.0678) (width 0.2032) (layer "B.Cu") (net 7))
 (segment (start 54.8152 57.8338) (end 54.8152 56.4692) (width 0.2032) (layer "F.Cu") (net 8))
 (segment (start 53.8336 58.8154) (end 54.8152 57.8338) (width 0.2032) (layer "F.Cu") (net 8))
 (segment (start 53.8336 60.3292) (end 53.8336 58.8154) (width 0.2032) (layer "F.Cu") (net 8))
 (via (at 54.8152 57.5569) (size 0.762) (drill 0.381) (layers "F.Cu" "B.Cu") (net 8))
 (segment (start 54.8152 55.7486) (end 54.7194 55.6528) (width 0.2032) (layer "B.Cu") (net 8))
 (segment (start 54.8152 57.5569) (end 54.8152 55.7486) (width 0.2032) (layer "B.Cu") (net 8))
 (segment (start 54.7194 55.6528) (end 54.232 55.6528) (width 0.2032) (layer "B.Cu") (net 8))
 (segment (start 55.0836 58.7966) (end 55.0836 60.3292) (width 0.2032) (layer "F.Cu") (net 3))
 (segment (start 56.3626 57.5176) (end 55.0836 58.7966) (width 0.2032) (layer "F.Cu") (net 3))
 (segment (start 55.4802 56.3042) (end 56.332257 56.3042) (width 0.2032) (layer "F.Cu") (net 3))
 (segment (start 56.332257 56.3042) (end 56.4014 56.373343) (width 0.2032) (layer "F.Cu") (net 3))
 (segment (start 56.4014 56.373343) (end 56.3638 56.335743) (width 0.2032) (layer "F.Cu") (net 3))
 (segment (start 56.3626 56.412143) (end 56.3626 57.5176) (width 0.2032) (layer "F.Cu") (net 3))
 (segment (start 56.4014 56.373343) (end 56.3626 56.412143) (width 0.2032) (layer "F.Cu") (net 3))
 (via (at 56.3638 56.335743) (size 0.762) (drill 0.381) (layers "F.Cu" "B.Cu") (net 3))
 (segment (start 53.3654 54.9656) (end 53.5526 55.1528) (width 0.2032) (layer "B.Cu") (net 3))
 (segment (start 56.234143 56.335743) (end 56.3638 56.335743) (width 0.2032) (layer "B.Cu") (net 3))
 (segment (start 54.232 52.6528) (end 53.6462 52.6528) (width 0.2032) (layer "B.Cu") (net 3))
 (segment (start 55.0512 55.1528) (end 56.234143 56.335743) (width 0.2032) (layer "B.Cu") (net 3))
 (segment (start 53.5526 55.1528) (end 54.232 55.1528) (width 0.2032) (layer "B.Cu") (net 3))
 (segment (start 53.3654 52.9336) (end 53.3654 54.9656) (width 0.2032) (layer "B.Cu") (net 3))
 (segment (start 54.232 55.1528) (end 55.0512 55.1528) (width 0.2032) (layer "B.Cu") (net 3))
 (segment (start 53.6462 52.6528) (end 53.3654 52.9336) (width 0.2032) (layer "B.Cu") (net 3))
 (segment (start 52.5728 54.8254) (end 52.5728 60.3292) (width 0.2032) (layer "B.Cu") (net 10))
 (segment (start 52.4002 54.6528) (end 52.5728 54.8254) (width 0.2032) (layer "B.Cu") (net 10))
 (segment (start 51.902 54.6528) (end 52.4002 54.6528) (width 0.2032) (layer "B.Cu") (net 10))
 (segment (start 54.6354 58.3184) (end 53.7972 59.1566) (width 0.2032) (layer "B.Cu") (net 9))
 (segment (start 55.6768 53.9242) (end 56.9976 53.9242) (width 0.2032) (layer "B.Cu") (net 9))
 (segment (start 53.7972 59.1566) (end 53.7972 60.3504) (width 0.2032) (layer "B.Cu") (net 9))
 (segment (start 54.9054 53.1528) (end 55.6768 53.9242) (width 0.2032) (layer "B.Cu") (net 9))
 (segment (start 56.388 58.3184) (end 54.6354 58.3184) (width 0.2032) (layer "B.Cu") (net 9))
 (segment (start 56.9976 53.9242) (end 57.2464 54.173) (width 0.2032) (layer "B.Cu") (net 9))
 (segment (start 54.232 53.1528) (end 54.9054 53.1528) (width 0.2032) (layer "B.Cu") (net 9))
 (segment (start 57.2464 57.46) (end 56.388 58.3184) (width 0.2032) (layer "B.Cu") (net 9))
 (segment (start 57.2464 54.173) (end 57.2464 57.46) (width 0.2032) (layer "B.Cu") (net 9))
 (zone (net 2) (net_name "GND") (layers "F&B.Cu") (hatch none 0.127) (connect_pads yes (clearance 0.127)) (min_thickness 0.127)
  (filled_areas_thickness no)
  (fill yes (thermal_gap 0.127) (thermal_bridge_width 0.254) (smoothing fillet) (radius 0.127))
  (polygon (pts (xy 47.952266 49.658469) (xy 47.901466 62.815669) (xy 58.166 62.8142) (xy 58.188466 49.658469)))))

